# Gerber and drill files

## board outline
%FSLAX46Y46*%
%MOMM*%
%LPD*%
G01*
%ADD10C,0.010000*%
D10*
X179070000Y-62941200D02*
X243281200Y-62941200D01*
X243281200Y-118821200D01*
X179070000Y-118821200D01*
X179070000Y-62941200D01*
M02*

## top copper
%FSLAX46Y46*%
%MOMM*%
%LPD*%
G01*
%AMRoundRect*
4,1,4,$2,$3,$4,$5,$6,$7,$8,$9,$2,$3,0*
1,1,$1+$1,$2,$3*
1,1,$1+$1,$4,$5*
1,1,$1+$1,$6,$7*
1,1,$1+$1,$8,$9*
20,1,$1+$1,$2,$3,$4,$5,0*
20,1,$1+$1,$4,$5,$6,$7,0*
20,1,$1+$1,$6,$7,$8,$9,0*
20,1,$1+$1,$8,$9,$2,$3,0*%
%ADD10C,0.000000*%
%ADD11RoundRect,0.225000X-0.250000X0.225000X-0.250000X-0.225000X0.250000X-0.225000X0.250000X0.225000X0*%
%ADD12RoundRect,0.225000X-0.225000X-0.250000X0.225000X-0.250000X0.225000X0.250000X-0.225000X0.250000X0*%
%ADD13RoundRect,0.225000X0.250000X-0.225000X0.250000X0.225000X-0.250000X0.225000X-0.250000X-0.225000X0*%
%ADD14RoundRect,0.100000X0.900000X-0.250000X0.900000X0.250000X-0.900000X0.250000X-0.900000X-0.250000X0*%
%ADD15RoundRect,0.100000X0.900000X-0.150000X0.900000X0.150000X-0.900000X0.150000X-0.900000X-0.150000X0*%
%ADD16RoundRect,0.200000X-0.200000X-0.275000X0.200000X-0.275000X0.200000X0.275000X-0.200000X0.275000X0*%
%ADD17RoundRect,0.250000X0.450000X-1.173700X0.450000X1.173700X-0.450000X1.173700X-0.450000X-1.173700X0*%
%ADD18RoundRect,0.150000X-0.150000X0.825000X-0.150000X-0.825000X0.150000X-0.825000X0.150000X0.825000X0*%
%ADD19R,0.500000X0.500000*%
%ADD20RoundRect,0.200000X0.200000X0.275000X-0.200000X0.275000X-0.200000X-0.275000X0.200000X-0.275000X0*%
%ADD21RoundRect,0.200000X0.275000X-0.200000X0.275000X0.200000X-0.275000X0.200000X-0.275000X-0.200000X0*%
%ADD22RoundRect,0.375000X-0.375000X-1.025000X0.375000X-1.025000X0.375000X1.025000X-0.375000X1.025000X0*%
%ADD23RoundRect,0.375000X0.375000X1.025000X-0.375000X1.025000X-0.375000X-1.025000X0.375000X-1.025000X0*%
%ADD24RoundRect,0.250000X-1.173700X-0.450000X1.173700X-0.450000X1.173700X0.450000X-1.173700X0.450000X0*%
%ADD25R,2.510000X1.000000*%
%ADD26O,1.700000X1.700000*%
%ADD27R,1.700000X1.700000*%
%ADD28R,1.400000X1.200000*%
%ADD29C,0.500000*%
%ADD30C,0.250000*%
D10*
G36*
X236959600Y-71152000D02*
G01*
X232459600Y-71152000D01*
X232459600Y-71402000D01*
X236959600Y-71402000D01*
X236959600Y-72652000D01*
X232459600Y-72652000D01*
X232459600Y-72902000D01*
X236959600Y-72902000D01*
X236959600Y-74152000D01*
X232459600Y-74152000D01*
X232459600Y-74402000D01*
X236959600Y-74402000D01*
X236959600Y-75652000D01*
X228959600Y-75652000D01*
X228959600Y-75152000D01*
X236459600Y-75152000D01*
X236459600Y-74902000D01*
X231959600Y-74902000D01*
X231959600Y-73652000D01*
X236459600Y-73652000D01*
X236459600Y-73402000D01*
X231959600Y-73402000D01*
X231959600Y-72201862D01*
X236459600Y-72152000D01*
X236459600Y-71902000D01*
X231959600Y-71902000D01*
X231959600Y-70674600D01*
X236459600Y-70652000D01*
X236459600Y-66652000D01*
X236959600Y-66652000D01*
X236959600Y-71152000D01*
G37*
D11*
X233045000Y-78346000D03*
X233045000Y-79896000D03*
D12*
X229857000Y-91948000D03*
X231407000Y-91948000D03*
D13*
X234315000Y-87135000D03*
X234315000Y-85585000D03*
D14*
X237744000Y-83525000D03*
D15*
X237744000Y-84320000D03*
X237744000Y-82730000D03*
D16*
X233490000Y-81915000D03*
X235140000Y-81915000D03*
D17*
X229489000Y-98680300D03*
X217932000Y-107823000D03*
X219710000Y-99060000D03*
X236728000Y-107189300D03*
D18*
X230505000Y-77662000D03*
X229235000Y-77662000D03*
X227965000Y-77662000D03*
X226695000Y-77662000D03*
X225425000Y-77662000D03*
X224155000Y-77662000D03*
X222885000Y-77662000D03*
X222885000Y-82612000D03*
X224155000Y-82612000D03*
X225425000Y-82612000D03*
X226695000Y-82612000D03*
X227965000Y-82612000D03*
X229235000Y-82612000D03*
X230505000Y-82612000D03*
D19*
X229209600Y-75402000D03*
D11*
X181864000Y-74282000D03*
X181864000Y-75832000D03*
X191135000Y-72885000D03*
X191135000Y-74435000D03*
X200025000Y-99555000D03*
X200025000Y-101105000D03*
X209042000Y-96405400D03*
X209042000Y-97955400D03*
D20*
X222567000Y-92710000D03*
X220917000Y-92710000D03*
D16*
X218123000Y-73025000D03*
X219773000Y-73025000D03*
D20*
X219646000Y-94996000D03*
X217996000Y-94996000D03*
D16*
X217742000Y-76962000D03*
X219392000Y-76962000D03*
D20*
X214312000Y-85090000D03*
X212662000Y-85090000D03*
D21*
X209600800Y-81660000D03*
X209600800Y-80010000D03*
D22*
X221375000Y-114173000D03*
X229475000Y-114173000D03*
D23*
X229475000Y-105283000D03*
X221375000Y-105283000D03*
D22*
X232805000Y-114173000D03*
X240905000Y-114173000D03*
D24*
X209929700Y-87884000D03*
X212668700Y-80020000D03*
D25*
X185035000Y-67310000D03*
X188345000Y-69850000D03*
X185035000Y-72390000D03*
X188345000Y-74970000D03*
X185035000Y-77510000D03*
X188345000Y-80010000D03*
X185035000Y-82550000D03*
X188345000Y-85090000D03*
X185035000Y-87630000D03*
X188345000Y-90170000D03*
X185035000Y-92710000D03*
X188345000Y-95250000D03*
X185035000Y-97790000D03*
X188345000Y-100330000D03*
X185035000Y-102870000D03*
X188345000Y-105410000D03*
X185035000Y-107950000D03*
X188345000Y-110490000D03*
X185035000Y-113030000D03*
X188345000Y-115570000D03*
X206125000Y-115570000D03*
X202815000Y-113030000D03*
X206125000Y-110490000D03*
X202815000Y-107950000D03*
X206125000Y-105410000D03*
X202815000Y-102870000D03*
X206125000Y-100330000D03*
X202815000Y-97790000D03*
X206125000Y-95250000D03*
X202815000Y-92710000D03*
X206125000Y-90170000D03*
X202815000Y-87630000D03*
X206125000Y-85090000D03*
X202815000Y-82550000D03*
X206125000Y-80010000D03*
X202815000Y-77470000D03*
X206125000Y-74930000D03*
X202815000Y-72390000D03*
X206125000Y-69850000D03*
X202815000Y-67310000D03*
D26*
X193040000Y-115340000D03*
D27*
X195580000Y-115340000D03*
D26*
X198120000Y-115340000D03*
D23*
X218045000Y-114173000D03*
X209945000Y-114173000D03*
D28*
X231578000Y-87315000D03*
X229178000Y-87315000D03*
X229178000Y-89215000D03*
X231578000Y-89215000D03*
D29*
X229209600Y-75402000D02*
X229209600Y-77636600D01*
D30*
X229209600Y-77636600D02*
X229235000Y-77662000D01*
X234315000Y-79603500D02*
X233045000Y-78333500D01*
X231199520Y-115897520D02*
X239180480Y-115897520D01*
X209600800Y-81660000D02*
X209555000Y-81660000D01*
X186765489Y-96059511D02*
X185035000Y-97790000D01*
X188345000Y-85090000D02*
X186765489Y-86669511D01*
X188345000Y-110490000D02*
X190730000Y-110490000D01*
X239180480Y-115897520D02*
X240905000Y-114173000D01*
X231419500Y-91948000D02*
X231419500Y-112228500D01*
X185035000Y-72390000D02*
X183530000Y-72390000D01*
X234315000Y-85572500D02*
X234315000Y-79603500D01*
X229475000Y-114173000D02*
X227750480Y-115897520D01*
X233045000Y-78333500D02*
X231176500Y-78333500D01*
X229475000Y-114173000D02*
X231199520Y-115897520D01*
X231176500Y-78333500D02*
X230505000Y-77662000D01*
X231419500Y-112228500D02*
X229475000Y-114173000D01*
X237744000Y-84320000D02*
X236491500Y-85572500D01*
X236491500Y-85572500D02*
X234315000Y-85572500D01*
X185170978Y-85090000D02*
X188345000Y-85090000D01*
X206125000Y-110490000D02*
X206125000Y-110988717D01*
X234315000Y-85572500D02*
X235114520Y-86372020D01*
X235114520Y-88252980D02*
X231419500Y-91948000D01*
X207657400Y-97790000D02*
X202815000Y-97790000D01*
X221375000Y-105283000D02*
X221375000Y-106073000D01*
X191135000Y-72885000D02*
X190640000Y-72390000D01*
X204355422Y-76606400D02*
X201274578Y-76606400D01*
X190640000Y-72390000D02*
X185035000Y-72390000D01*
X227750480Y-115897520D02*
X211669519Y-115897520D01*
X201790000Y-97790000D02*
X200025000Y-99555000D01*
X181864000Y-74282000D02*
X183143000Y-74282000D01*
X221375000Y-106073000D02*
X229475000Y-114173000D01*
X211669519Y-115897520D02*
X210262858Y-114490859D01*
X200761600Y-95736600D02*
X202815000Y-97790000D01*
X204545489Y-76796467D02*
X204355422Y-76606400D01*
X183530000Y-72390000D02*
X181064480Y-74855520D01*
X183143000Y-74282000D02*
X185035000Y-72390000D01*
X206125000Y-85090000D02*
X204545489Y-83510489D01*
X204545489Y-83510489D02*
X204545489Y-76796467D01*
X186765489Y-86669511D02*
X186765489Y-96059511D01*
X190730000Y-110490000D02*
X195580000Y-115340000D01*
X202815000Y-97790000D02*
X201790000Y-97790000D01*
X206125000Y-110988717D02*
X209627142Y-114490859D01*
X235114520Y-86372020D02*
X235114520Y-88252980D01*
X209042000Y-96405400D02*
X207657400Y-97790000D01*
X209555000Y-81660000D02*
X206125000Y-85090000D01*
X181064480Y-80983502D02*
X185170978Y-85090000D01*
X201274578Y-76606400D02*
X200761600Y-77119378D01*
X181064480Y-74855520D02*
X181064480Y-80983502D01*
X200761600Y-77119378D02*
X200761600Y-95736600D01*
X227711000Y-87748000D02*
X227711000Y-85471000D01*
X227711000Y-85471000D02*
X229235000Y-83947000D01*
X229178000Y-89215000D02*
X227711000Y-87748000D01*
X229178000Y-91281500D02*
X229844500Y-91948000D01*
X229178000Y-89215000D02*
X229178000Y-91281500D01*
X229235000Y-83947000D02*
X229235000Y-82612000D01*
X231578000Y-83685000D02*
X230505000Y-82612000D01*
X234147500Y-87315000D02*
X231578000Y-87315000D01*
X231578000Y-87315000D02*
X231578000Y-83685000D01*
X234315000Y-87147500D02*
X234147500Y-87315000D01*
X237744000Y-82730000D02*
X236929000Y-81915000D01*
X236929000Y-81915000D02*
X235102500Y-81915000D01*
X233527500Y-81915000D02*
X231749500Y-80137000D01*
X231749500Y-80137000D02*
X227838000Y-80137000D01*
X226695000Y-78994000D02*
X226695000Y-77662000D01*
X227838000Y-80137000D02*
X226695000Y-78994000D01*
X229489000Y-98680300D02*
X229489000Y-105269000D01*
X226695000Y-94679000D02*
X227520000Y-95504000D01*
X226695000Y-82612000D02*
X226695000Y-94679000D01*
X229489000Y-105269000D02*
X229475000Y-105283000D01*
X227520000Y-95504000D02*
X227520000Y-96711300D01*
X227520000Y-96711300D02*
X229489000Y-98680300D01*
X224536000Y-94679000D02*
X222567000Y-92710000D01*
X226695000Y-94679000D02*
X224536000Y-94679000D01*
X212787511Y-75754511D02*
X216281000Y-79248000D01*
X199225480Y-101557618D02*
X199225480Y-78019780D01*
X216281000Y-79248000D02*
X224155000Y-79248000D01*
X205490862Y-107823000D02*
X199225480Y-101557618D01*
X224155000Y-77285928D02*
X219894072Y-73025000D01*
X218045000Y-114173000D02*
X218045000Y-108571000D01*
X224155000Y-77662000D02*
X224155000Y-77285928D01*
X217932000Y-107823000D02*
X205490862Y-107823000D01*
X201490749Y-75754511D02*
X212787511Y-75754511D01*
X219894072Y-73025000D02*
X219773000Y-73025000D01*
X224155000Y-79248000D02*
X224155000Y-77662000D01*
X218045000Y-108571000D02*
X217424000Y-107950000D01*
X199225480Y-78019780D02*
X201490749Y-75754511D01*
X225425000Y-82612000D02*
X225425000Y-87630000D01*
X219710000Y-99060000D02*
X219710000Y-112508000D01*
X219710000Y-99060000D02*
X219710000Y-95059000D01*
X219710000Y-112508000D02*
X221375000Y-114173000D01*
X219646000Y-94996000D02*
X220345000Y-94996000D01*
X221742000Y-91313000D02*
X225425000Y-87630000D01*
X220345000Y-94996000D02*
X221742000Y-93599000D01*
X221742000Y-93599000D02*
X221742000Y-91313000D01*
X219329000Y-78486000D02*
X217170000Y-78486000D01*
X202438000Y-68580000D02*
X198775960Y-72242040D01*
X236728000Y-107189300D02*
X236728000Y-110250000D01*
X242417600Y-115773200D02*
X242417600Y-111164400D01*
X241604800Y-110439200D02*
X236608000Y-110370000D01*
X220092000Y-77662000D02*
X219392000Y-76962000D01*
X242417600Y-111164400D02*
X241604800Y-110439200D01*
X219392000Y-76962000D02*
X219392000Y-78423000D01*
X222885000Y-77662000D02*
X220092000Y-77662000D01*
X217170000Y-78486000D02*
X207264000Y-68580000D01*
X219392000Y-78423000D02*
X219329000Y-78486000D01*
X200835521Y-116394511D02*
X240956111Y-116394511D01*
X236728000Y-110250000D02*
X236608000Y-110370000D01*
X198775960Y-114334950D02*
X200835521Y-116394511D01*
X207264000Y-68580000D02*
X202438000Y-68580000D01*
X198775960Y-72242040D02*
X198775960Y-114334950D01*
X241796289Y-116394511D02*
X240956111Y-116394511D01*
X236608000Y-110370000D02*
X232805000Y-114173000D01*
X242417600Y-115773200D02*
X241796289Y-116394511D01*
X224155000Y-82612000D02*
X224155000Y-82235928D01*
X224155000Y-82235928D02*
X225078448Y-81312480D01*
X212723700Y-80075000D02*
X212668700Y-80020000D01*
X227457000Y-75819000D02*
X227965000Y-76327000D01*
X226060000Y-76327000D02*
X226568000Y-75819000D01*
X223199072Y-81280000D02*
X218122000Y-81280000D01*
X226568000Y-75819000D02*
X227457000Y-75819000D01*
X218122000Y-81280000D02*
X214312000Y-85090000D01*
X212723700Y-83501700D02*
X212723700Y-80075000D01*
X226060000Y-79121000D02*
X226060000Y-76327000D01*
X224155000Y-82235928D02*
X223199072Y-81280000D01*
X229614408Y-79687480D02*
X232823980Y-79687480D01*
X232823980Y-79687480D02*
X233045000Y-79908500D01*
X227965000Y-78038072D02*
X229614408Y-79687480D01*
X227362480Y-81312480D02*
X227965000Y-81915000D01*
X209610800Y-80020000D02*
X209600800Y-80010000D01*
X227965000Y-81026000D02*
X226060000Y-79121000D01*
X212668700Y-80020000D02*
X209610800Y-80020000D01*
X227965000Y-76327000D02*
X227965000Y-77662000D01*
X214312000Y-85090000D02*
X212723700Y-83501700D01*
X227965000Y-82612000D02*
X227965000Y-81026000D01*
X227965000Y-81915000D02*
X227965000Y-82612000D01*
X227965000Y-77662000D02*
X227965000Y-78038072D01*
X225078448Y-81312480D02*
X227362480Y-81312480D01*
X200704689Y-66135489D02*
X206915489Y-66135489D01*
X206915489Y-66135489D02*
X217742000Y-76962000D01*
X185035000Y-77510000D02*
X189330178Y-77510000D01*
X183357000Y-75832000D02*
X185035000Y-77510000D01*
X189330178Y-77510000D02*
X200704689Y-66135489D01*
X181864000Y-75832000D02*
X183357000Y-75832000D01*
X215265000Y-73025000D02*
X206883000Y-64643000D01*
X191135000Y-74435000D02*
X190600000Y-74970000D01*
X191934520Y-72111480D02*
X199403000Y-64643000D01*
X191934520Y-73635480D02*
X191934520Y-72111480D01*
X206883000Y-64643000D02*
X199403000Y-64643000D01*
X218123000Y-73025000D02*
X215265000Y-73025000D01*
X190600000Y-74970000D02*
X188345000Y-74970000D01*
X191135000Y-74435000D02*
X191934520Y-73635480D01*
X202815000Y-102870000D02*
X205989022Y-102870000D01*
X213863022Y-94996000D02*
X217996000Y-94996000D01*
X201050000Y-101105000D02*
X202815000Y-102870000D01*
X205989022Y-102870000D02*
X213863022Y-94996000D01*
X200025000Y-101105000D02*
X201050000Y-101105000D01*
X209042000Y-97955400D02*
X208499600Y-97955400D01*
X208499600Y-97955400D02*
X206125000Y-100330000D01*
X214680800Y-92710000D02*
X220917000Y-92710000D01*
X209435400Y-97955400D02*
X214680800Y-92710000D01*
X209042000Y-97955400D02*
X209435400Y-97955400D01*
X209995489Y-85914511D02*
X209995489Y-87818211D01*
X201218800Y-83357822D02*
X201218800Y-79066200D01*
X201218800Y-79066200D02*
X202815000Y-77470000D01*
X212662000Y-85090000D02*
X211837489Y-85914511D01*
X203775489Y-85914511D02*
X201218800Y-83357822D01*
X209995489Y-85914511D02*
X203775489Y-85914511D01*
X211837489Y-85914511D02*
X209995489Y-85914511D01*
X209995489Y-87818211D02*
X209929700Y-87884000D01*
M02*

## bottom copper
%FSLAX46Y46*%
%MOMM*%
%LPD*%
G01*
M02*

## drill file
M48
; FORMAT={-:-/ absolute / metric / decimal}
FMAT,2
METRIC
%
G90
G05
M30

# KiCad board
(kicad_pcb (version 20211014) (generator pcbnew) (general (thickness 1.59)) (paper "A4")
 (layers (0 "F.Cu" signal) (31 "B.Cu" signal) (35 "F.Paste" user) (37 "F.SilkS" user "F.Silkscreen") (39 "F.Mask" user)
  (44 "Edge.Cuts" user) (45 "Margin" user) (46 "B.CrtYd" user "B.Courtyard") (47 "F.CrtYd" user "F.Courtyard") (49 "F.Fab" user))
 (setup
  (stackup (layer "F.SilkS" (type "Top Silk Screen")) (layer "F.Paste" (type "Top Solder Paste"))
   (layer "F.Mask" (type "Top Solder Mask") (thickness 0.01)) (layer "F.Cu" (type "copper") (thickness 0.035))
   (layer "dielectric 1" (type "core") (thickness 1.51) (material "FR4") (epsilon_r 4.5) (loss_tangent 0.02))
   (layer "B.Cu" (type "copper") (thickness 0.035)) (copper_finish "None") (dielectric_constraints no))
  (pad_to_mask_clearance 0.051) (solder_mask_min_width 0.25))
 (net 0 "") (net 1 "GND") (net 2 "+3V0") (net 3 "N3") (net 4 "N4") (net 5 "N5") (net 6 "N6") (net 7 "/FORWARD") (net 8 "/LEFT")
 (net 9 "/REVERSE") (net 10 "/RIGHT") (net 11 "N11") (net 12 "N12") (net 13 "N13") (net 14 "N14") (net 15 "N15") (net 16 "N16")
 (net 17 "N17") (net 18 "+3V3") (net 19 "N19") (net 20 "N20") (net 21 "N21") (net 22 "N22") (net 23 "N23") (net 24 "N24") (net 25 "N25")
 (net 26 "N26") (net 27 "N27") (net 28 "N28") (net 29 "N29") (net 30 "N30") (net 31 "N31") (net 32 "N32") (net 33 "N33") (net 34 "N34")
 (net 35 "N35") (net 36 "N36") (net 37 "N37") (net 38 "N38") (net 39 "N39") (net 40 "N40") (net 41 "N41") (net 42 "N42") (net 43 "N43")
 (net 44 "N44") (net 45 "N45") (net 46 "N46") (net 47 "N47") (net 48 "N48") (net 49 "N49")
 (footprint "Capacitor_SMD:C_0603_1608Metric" (layer "F.Cu") (at 233.045 79.121 -90)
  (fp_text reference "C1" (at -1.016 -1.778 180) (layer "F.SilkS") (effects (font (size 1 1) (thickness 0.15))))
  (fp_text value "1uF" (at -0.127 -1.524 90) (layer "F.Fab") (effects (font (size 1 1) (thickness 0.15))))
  (pad "1" smd roundrect locked (at -0.775 0 270) (size 0.9 0.95) (layers "F.Cu" "F.Paste" "F.Mask") (roundrect_rratio 0.25) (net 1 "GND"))
  (pad "2" smd roundrect locked (at 0.775 0 270) (size 0.9 0.95) (layers "F.Cu" "F.Paste" "F.Mask") (roundrect_rratio 0.25) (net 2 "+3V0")))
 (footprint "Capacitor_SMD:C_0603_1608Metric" (layer "F.Cu") (at 230.632 91.948)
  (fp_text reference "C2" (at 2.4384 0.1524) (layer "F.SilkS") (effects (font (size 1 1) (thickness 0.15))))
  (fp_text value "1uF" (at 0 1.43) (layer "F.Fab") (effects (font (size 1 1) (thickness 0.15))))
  (pad "1" smd roundrect locked (at -0.775 0) (size 0.9 0.95) (layers "F.Cu" "F.Paste" "F.Mask") (roundrect_rratio 0.25) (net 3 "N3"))
  (pad "2" smd roundrect locked (at 0.775 0) (size 0.9 0.95) (layers "F.Cu" "F.Paste" "F.Mask") (roundrect_rratio 0.25) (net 1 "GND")))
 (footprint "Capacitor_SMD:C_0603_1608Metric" (layer "F.Cu") (at 234.315 86.36 90)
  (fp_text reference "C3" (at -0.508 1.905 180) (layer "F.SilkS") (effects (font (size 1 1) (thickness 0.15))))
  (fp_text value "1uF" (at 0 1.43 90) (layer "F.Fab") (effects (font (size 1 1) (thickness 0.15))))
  (pad "1" smd roundrect locked (at -0.775 0 90) (size 0.9 0.95) (layers "F.Cu" "F.Paste" "F.Mask") (roundrect_rratio 0.25) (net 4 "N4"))
  (pad "2" smd roundrect locked (at 0.775 0 90) (size 0.9 0.95) (layers "F.Cu" "F.Paste" "F.Mask") (roundrect_rratio 0.25) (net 1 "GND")))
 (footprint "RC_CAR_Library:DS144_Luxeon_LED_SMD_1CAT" (layer "F.Cu") (at 237.744 83.525 90)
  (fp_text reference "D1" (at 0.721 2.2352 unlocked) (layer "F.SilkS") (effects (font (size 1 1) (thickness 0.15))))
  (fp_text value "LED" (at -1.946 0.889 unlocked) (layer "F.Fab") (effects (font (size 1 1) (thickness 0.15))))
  (pad "" smd roundrect (at 0 0 90) (size 0.7 2) (layers "F.Cu" "F.Paste" "F.Mask") (roundrect_rratio 0.1428571429) (zone_connect 1))
  (pad "1" smd roundrect (at -0.795 0 90) (size 0.5 2) (layers "F.Cu" "F.Paste" "F.Mask") (roundrect_rratio 0.2) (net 1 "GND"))
  (pad "2" smd roundrect (at 0.795 0 90) (size 0.5 2) (layers "F.Cu" "F.Paste" "F.Mask") (roundrect_rratio 0.2) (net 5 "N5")))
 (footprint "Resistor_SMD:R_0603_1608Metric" (layer "F.Cu") (at 234.315 81.915)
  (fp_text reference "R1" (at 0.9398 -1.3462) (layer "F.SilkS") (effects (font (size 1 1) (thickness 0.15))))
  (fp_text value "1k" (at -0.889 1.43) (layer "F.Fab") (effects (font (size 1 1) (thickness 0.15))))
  (pad "1" smd roundrect locked (at -0.825 0) (size 0.8 0.95) (layers "F.Cu" "F.Paste" "F.Mask") (roundrect_rratio 0.25) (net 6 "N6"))
  (pad "2" smd roundrect locked (at 0.825 0) (size 0.8 0.95) (layers "F.Cu" "F.Paste" "F.Mask") (roundrect_rratio 0.25) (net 5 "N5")))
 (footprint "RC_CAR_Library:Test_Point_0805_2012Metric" (layer "F.Cu") (at 229.489 98.679 90)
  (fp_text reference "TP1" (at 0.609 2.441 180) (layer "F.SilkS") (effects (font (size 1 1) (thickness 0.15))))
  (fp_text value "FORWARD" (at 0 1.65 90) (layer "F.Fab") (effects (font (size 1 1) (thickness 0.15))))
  (pad "1" smd roundrect (at -0.0013 0 90) (size 2.8474 1.4) (layers "F.Cu" "F.Paste" "F.Mask") (roundrect_rratio 0.1785714286)
   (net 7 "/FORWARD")))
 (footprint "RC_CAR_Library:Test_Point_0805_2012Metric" (layer "F.Cu") (at 217.932 107.8217 90)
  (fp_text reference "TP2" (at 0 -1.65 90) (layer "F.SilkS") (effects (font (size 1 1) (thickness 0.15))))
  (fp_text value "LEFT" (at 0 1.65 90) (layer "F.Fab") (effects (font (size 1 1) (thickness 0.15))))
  (pad "1" smd roundrect (at -0.0013 0 90) (size 2.8474 1.4) (layers "F.Cu" "F.Paste" "F.Mask") (roundrect_rratio 0.1785714286)
   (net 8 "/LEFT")))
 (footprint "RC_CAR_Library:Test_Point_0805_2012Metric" (layer "F.Cu") (at 219.71 99.0587 90)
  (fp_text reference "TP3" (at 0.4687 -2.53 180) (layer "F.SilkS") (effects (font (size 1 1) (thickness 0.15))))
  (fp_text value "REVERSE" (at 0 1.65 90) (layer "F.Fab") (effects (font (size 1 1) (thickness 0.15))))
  (pad "1" smd roundrect (at -0.0013 0 90) (size 2.8474 1.4) (layers "F.Cu" "F.Paste" "F.Mask") (roundrect_rratio 0.1785714286)
   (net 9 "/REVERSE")))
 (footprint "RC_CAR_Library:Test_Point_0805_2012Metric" (layer "F.Cu") (at 236.728 107.188 90)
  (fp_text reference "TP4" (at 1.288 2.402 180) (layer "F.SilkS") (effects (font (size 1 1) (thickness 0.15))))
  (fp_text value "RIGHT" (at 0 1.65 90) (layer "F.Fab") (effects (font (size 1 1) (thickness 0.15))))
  (pad "1" smd roundrect (at -0.0013 0 90) (size 2.8474 1.4) (layers "F.Cu" "F.Paste" "F.Mask") (roundrect_rratio 0.1785714286)
   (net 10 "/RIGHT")))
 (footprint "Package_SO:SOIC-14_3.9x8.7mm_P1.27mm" (layer "F.Cu") (at 226.695 80.137 -90)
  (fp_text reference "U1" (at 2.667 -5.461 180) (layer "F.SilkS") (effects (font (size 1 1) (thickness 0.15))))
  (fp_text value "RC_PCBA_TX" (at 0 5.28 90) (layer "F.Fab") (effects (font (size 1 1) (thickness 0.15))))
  (pad "1" smd roundrect locked (at -2.475 -3.81 270) (size 1.95 0.6) (layers "F.Cu" "F.Paste" "F.Mask") (roundrect_rratio 0.25)
   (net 1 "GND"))
  (pad "2" smd roundrect locked (at -2.475 -2.54 270) (size 1.95 0.6) (layers "F.Cu" "F.Paste" "F.Mask") (roundrect_rratio 0.25)
   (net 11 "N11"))
  (pad "3" smd roundrect locked (at -2.475 -1.27 270) (size 1.95 0.6) (layers "F.Cu" "F.Paste" "F.Mask") (roundrect_rratio 0.25)
   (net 2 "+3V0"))
  (pad "4" smd roundrect locked (at -2.475 0 270) (size 1.95 0.6) (layers "F.Cu" "F.Paste" "F.Mask") (roundrect_rratio 0.25) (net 6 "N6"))
  (pad "5" smd roundrect locked (at -2.475 1.27 270) (size 1.95 0.6) (layers "F.Cu" "F.Paste" "F.Mask") (roundrect_rratio 0.25)
   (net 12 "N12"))
  (pad "6" smd roundrect locked (at -2.475 2.54 270) (size 1.95 0.6) (layers "F.Cu" "F.Paste" "F.Mask") (roundrect_rratio 0.25)
   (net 8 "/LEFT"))
  (pad "7" smd roundrect locked (at -2.475 3.81 270) (size 1.95 0.6) (layers "F.Cu" "F.Paste" "F.Mask") (roundrect_rratio 0.25)
   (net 10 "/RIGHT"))
  (pad "8" smd roundrect locked (at 2.475 3.81 270) (size 1.95 0.6) (layers "F.Cu" "F.Paste" "F.Mask") (roundrect_rratio 0.25)
   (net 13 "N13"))
  (pad "9" smd roundrect locked (at 2.475 2.54 270) (size 1.95 0.6) (layers "F.Cu" "F.Paste" "F.Mask") (roundrect_rratio 0.25)
   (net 2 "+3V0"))
  (pad "10" smd roundrect locked (at 2.475 1.27 270) (size 1.95 0.6) (layers "F.Cu" "F.Paste" "F.Mask") (roundrect_rratio 0.25)
   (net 9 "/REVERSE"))
  (pad "11" smd roundrect locked (at 2.475 0 270) (size 1.95 0.6) (layers "F.Cu" "F.Paste" "F.Mask") (roundrect_rratio 0.25)
   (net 7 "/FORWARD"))
  (pad "12" smd roundrect locked (at 2.475 -1.27 270) (size 1.95 0.6) (layers "F.Cu" "F.Paste" "F.Mask") (roundrect_rratio 0.25)
   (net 2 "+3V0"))
  (pad "13" smd roundrect locked (at 2.475 -2.54 270) (size 1.95 0.6) (layers "F.Cu" "F.Paste" "F.Mask") (roundrect_rratio 0.25)
   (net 3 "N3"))
  (pad "14" smd roundrect locked (at 2.475 -3.81 270) (size 1.95 0.6) (layers "F.Cu" "F.Paste" "F.Mask") (roundrect_rratio 0.25)
   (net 4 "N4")))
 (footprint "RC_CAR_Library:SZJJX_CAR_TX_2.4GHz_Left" (layer "F.Cu") (at 229.2096 73.152 -90)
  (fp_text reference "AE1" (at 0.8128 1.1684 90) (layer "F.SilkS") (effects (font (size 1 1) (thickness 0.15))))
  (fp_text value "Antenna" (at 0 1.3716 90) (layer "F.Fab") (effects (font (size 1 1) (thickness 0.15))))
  (fp_poly
   (pts (xy -2 -7.75) (xy -2 -3.25) (xy -1.75 -3.25) (xy -1.75 -7.75) (xy -0.5 -7.75) (xy -0.5 -3.25) (xy -0.25 -3.25) (xy -0.25 -7.75)
    (xy 1 -7.75) (xy 1 -3.25) (xy 1.25 -3.25) (xy 1.25 -7.75) (xy 2.5 -7.75) (xy 2.5 0.25) (xy 2 0.25) (xy 2 -7.25) (xy 1.75 -7.25)
    (xy 1.75 -2.75) (xy 0.5 -2.75) (xy 0.5 -7.25) (xy 0.25 -7.25) (xy 0.25 -2.75) (xy -0.950138 -2.75) (xy -1 -7.25) (xy -1.25 -7.25)
    (xy -1.25 -2.75) (xy -2.4774 -2.75) (xy -2.5 -7.25) (xy -6.5 -7.25) (xy -6.5 -7.75))
   (layer "F.Cu") (width 0) (fill solid))
  (pad "1" connect rect (at 2.25 0 270) (size 0.5 0.5) (layers "F.Cu") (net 11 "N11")))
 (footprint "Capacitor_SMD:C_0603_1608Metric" (layer "F.Cu") (at 181.864 75.057 -90)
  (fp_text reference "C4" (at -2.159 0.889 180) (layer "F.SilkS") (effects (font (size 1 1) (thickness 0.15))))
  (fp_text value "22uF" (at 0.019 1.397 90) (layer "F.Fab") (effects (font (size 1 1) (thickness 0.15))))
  (pad "1" smd roundrect locked (at -0.775 0 270) (size 0.9 0.95) (layers "F.Cu" "F.Paste" "F.Mask") (roundrect_rratio 0.25) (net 1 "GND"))
  (pad "2" smd roundrect locked (at 0.775 0 270) (size 0.9 0.95) (layers "F.Cu" "F.Paste" "F.Mask") (roundrect_rratio 0.25) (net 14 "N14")))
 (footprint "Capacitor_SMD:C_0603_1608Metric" (layer "F.Cu") (at 191.135 73.66 -90)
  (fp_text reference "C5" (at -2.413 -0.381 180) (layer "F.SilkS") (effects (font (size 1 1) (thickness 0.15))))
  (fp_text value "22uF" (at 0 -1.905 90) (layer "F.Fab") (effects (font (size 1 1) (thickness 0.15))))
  (pad "1" smd roundrect locked (at -0.775 0 270) (size 0.9 0.95) (layers "F.Cu" "F.Paste" "F.Mask") (roundrect_rratio 0.25) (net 1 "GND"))
  (pad "2" smd roundrect locked (at 0.775 0 270) (size 0.9 0.95) (layers "F.Cu" "F.Paste" "F.Mask") (roundrect_rratio 0.25) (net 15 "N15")))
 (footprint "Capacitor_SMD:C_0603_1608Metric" (layer "F.Cu") (at 200.025 100.33 -90)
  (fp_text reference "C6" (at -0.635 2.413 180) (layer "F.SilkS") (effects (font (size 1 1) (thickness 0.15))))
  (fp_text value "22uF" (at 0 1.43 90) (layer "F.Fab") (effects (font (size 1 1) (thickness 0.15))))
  (pad "1" smd roundrect locked (at -0.775 0 270) (size 0.9 0.95) (layers "F.Cu" "F.Paste" "F.Mask") (roundrect_rratio 0.25) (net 1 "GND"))
  (pad "2" smd roundrect locked (at 0.775 0 270) (size 0.9 0.95) (layers "F.Cu" "F.Paste" "F.Mask") (roundrect_rratio 0.25) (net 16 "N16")))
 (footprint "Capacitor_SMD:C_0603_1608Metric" (layer "F.Cu") (at 209.042 97.1804 -90)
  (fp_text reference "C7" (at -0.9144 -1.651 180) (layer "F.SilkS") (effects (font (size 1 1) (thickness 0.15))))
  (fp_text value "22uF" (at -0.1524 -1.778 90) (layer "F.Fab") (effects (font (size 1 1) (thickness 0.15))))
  (pad "1" smd roundrect locked (at -0.775 0 270) (size 0.9 0.95) (layers "F.Cu" "F.Paste" "F.Mask") (roundrect_rratio 0.25) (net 1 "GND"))
  (pad "2" smd roundrect locked (at 0.775 0 270) (size 0.9 0.95) (layers "F.Cu" "F.Paste" "F.Mask") (roundrect_rratio 0.25) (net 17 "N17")))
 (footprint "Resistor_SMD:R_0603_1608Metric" (layer "F.Cu") (at 221.742 92.71 180)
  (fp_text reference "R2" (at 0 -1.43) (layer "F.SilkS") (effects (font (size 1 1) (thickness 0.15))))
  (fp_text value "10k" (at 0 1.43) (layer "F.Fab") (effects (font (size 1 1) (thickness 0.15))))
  (pad "1" smd roundrect locked (at -0.825 0 180) (size 0.8 0.95) (layers "F.Cu" "F.Paste" "F.Mask") (roundrect_rratio 0.25)
   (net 7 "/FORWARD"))
  (pad "2" smd roundrect locked (at 0.825 0 180) (size 0.8 0.95) (layers "F.Cu" "F.Paste" "F.Mask") (roundrect_rratio 0.25) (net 17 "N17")))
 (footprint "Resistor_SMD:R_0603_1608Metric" (layer "F.Cu") (at 218.948 73.025)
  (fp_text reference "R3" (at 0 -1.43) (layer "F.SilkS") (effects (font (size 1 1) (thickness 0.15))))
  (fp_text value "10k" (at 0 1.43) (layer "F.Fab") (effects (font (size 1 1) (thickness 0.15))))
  (pad "1" smd roundrect locked (at -0.825 0) (size 0.8 0.95) (layers "F.Cu" "F.Paste" "F.Mask") (roundrect_rratio 0.25) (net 15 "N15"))
  (pad "2" smd roundrect locked (at 0.825 0) (size 0.8 0.95) (layers "F.Cu" "F.Paste" "F.Mask") (roundrect_rratio 0.25) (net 8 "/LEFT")))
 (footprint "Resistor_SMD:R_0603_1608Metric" (layer "F.Cu") (at 218.821 94.996 180)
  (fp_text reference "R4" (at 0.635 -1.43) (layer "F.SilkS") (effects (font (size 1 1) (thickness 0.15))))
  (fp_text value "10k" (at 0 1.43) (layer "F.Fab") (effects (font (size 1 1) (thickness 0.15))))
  (pad "1" smd roundrect locked (at -0.825 0 180) (size 0.8 0.95) (layers "F.Cu" "F.Paste" "F.Mask") (roundrect_rratio 0.25)
   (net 9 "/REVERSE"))
  (pad "2" smd roundrect locked (at 0.825 0 180) (size 0.8 0.95) (layers "F.Cu" "F.Paste" "F.Mask") (roundrect_rratio 0.25) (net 16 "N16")))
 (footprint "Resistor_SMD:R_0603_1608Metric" (layer "F.Cu") (at 218.567 76.962)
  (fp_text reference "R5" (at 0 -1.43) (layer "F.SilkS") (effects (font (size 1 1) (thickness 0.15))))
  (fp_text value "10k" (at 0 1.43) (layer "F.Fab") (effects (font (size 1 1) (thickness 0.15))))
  (pad "1" smd roundrect locked (at -0.825 0) (size 0.8 0.95) (layers "F.Cu" "F.Paste" "F.Mask") (roundrect_rratio 0.25) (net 14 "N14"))
  (pad "2" smd roundrect locked (at 0.825 0) (size 0.8 0.95) (layers "F.Cu" "F.Paste" "F.Mask") (roundrect_rratio 0.25) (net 10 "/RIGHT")))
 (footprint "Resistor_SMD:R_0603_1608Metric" (layer "F.Cu") (at 213.487 85.09 180)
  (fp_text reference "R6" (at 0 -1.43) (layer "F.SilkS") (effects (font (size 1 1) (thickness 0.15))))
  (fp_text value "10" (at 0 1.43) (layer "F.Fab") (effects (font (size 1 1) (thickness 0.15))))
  (pad "1" smd roundrect locked (at -0.825 0 180) (size 0.8 0.95) (layers "F.Cu" "F.Paste" "F.Mask") (roundrect_rratio 0.25) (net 2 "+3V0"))
  (pad "2" smd roundrect locked (at 0.825 0 180) (size 0.8 0.95) (layers "F.Cu" "F.Paste" "F.Mask") (roundrect_rratio 0.25) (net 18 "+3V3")))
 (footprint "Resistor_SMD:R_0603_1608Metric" (layer "F.Cu") (at 209.6008 80.835 90)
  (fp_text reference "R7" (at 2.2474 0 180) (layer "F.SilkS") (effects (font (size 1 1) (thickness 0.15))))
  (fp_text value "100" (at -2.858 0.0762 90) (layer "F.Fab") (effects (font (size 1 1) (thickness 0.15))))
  (pad "1" smd roundrect locked (at -0.825 0 90) (size 0.8 0.95) (layers "F.Cu" "F.Paste" "F.Mask") (roundrect_rratio 0.25) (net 1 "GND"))
  (pad "2" smd roundrect locked (at 0.825 0 90) (size 0.8 0.95) (layers "F.Cu" "F.Paste" "F.Mask") (roundrect_rratio 0.25) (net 2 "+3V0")))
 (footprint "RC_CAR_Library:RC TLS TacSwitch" (layer "F.Cu") (at 225.425 114.173)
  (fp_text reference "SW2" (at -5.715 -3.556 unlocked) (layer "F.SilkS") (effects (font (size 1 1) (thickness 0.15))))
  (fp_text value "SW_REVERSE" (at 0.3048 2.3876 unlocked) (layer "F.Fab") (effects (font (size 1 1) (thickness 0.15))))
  (pad "1" smd roundrect (at -4.05 0) (size 1.5 2.8) (layers "F.Cu" "F.Paste" "F.Mask") (roundrect_rratio 0.25) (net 9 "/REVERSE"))
  (pad "2" smd roundrect (at 4.05 0) (size 1.5 2.8) (layers "F.Cu" "F.Paste" "F.Mask") (roundrect_rratio 0.25) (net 1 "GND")))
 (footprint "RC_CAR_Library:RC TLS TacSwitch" (layer "F.Cu") (at 225.425 105.283 180)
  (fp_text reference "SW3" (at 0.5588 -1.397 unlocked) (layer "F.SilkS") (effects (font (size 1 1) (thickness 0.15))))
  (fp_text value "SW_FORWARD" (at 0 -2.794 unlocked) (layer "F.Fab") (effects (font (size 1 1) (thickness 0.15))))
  (pad "1" smd roundrect (at -4.05 0 180) (size 1.5 2.8) (layers "F.Cu" "F.Paste" "F.Mask") (roundrect_rratio 0.25) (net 7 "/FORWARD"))
  (pad "2" smd roundrect (at 4.05 0 180) (size 1.5 2.8) (layers "F.Cu" "F.Paste" "F.Mask") (roundrect_rratio 0.25) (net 1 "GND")))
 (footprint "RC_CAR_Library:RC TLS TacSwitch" (layer "F.Cu") (at 236.855 114.173)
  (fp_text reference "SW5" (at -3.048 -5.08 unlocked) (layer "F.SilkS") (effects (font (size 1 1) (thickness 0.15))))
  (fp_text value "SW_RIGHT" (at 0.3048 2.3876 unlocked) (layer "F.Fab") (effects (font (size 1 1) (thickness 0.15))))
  (pad "1" smd roundrect (at -4.05 0) (size 1.5 2.8) (layers "F.Cu" "F.Paste" "F.Mask") (roundrect_rratio 0.25) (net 10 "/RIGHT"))
  (pad "2" smd roundrect (at 4.05 0) (size 1.5 2.8) (layers "F.Cu" "F.Paste" "F.Mask") (roundrect_rratio 0.25) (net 1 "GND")))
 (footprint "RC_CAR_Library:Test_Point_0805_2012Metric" (layer "F.Cu") (at 209.931 87.884)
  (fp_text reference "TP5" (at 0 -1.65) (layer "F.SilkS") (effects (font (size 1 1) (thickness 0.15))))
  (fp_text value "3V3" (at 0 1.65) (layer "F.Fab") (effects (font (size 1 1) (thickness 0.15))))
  (pad "1" smd roundrect (at -0.0013 0) (size 2.8474 1.4) (layers "F.Cu" "F.Paste" "F.Mask") (roundrect_rratio 0.1785714286) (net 18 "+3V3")))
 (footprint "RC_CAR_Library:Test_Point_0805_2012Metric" (layer "F.Cu") (at 212.67 80.02)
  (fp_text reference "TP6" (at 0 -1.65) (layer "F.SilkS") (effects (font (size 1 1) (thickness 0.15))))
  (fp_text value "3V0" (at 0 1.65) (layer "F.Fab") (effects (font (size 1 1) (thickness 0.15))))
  (pad "1" smd roundrect (at -0.0013 0) (size 2.8474 1.4) (layers "F.Cu" "F.Paste" "F.Mask") (roundrect_rratio 0.1785714286) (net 2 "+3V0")))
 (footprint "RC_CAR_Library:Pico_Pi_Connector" (layer "F.Cu") (at 195.58 91.44)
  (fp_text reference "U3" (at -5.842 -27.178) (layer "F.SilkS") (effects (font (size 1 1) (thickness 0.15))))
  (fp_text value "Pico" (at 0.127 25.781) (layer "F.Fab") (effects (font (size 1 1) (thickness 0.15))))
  (pad "1" smd rect (at -10.545 -24.13) (size 2.51 1) (layers "F.Cu" "F.Paste" "F.Mask") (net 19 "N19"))
  (pad "2" smd rect (at -7.235 -21.59) (size 2.51 1) (layers "F.Cu" "F.Paste" "F.Mask") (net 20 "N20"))
  (pad "3" smd rect (at -10.545 -19.05) (size 2.51 1) (layers "F.Cu" "F.Paste" "F.Mask") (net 1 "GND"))
  (pad "4" smd rect (at -7.235 -16.47) (size 2.51 1) (layers "F.Cu" "F.Paste" "F.Mask") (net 15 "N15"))
  (pad "5" smd rect (at -10.545 -13.93) (size 2.51 1) (layers "F.Cu" "F.Paste" "F.Mask") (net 14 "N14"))
  (pad "6" smd rect (at -7.235 -11.43) (size 2.51 1) (layers "F.Cu" "F.Paste" "F.Mask") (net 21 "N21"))
  (pad "7" smd rect (at -10.545 -8.89) (size 2.51 1) (layers "F.Cu" "F.Paste" "F.Mask") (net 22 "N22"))
  (pad "8" smd rect (at -7.235 -6.35) (size 2.51 1) (layers "F.Cu" "F.Paste" "F.Mask") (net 1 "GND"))
  (pad "9" smd rect (at -10.545 -3.81) (size 2.51 1) (layers "F.Cu" "F.Paste" "F.Mask") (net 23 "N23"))
  (pad "10" smd rect (at -7.235 -1.27) (size 2.51 1) (layers "F.Cu" "F.Paste" "F.Mask") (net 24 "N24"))
  (pad "11" smd rect (at -10.545 1.27) (size 2.51 1) (layers "F.Cu" "F.Paste" "F.Mask") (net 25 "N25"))
  (pad "12" smd rect (at -7.235 3.81) (size 2.51 1) (layers "F.Cu" "F.Paste" "F.Mask") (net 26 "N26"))
  (pad "13" smd rect (at -10.545 6.35) (size 2.51 1) (layers "F.Cu" "F.Paste" "F.Mask") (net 1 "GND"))
  (pad "14" smd rect (at -7.235 8.89) (size 2.51 1) (layers "F.Cu" "F.Paste" "F.Mask") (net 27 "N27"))
  (pad "15" smd rect (at -10.545 11.43) (size 2.51 1) (layers "F.Cu" "F.Paste" "F.Mask") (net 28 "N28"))
  (pad "16" smd rect (at -7.235 13.97) (size 2.51 1) (layers "F.Cu" "F.Paste" "F.Mask") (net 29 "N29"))
  (pad "17" smd rect (at -10.545 16.51) (size 2.51 1) (layers "F.Cu" "F.Paste" "F.Mask") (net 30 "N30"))
  (pad "18" smd rect (at -7.235 19.05) (size 2.51 1) (layers "F.Cu" "F.Paste" "F.Mask") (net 1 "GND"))
  (pad "19" smd rect (at -10.545 21.59) (size 2.51 1) (layers "F.Cu" "F.Paste" "F.Mask") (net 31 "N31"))
  (pad "20" smd rect (at -7.235 24.13) (size 2.51 1) (layers "F.Cu" "F.Paste" "F.Mask") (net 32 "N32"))
  (pad "21" smd rect (at 10.545 24.13) (size 2.51 1) (layers "F.Cu" "F.Paste" "F.Mask") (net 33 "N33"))
  (pad "22" smd rect (at 7.235 21.59) (size 2.51 1) (layers "F.Cu" "F.Paste" "F.Mask") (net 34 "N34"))
  (pad "23" smd rect (at 10.545 19.05) (size 2.51 1) (layers "F.Cu" "F.Paste" "F.Mask") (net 1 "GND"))
  (pad "24" smd rect (at 7.235 16.51) (size 2.51 1) (layers "F.Cu" "F.Paste" "F.Mask") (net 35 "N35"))
  (pad "25" smd rect (at 10.545 13.97) (size 2.51 1) (layers "F.Cu" "F.Paste" "F.Mask") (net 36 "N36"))
  (pad "26" smd rect (at 7.235 11.43) (size 2.51 1) (layers "F.Cu" "F.Paste" "F.Mask") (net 16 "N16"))
  (pad "27" smd rect (at 10.545 8.89) (size 2.51 1) (layers "F.Cu" "F.Paste" "F.Mask") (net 17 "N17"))
  (pad "28" smd rect (at 7.235 6.35) (size 2.51 1) (layers "F.Cu" "F.Paste" "F.Mask") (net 1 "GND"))
  (pad "29" smd rect (at 10.545 3.81) (size 2.51 1) (layers "F.Cu" "F.Paste" "F.Mask") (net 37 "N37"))
  (pad "30" smd rect (at 7.235 1.27) (size 2.51 1) (layers "F.Cu" "F.Paste" "F.Mask") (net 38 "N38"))
  (pad "31" smd rect (at 10.545 -1.27) (size 2.51 1) (layers "F.Cu" "F.Paste" "F.Mask") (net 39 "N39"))
  (pad "32" smd rect (at 7.235 -3.81) (size 2.51 1) (layers "F.Cu" "F.Paste" "F.Mask") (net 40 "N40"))
  (pad "33" smd rect (at 10.545 -6.35) (size 2.51 1) (layers "F.Cu" "F.Paste" "F.Mask") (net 1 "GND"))
  (pad "34" smd rect (at 7.235 -8.89) (size 2.51 1) (layers "F.Cu" "F.Paste" "F.Mask") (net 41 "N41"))
  (pad "35" smd rect (at 10.545 -11.43) (size 2.51 1) (layers "F.Cu" "F.Paste" "F.Mask") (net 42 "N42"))
  (pad "36" smd rect (at 7.235 -13.97) (size 2.51 1) (layers "F.Cu" "F.Paste" "F.Mask") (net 18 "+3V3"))
  (pad "37" smd rect (at 10.545 -16.51) (size 2.51 1) (layers "F.Cu" "F.Paste" "F.Mask") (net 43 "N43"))
  (pad "38" smd rect (at 7.235 -19.05) (size 2.51 1) (layers "F.Cu" "F.Paste" "F.Mask") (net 1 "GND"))
  (pad "39" smd rect (at 10.545 -21.59) (size 2.51 1) (layers "F.Cu" "F.Paste" "F.Mask") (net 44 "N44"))
  (pad "40" smd rect (at 7.235 -24.13) (size 2.51 1) (layers "F.Cu" "F.Paste" "F.Mask") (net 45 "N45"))
  (pad "41" smd oval (at -2.54 23.9) (size 1.7 1.7) (layers "F.Cu" "F.Paste" "F.Mask") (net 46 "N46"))
  (pad "42" smd rect (at 0 23.9) (size 1.7 1.7) (layers "F.Cu" "F.Paste" "F.Mask") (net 1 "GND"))
  (pad "43" smd oval (at 2.54 23.9) (size 1.7 1.7) (layers "F.Cu" "F.Paste" "F.Mask") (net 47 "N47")))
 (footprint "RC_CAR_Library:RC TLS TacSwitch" (layer "F.Cu") (at 213.995 114.173 180)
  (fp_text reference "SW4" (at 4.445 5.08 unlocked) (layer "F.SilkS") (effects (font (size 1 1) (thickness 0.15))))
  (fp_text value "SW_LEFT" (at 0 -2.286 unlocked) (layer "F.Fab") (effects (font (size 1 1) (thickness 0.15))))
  (pad "1" smd roundrect (at -4.05 0 180) (size 1.5 2.8) (layers "F.Cu" "F.Paste" "F.Mask") (roundrect_rratio 0.25) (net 8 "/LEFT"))
  (pad "2" smd roundrect (at 4.05 0 180) (size 1.5 2.8) (layers "F.Cu" "F.Paste" "F.Mask") (roundrect_rratio 0.25) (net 1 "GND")))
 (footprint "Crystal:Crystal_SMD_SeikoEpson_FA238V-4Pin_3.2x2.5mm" (layer "F.Cu") (at 230.378 88.265 180)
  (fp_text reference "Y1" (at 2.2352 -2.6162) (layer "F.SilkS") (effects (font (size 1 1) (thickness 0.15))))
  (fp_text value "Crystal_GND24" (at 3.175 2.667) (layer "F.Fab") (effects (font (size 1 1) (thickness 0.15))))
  (pad "1" smd rect locked (at -1.2 0.95 180) (size 1.4 1.2) (layers "F.Cu" "F.Paste" "F.Mask") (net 4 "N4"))
  (pad "2" smd rect locked (at 1.2 0.95 180) (size 1.4 1.2) (layers "F.Cu" "F.Paste" "F.Mask") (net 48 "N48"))
  (pad "3" smd rect locked (at 1.2 -0.95 180) (size 1.4 1.2) (layers "F.Cu" "F.Paste" "F.Mask") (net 3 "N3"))
  (pad "4" smd rect locked (at -1.2 -0.95 180) (size 1.4 1.2) (layers "F.Cu" "F.Paste" "F.Mask") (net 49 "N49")))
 (gr_rect (start 179.07 62.9412) (end 243.2812 118.8212) (layer "Edge.Cuts") (width 0.01) (fill none))
 (segment (start 229.2096 75.402) (end 229.2096 77.6366) (width 0.5) (layer "F.Cu") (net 11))
 (segment (start 229.2096 77.6366) (end 229.235 77.662) (width 0.25) (layer "F.Cu") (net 11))
 (segment (start 234.315 79.6035) (end 233.045 78.3335) (width 0.25) (layer "F.Cu") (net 1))
 (segment (start 231.19952 115.89752) (end 239.18048 115.89752) (width 0.25) (layer "F.Cu") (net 1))
 (segment (start 209.6008 81.66) (end 209.555 81.66) (width 0.25) (layer "F.Cu") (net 1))
 (segment (start 186.765489 96.059511) (end 185.035 97.79) (width 0.25) (layer "F.Cu") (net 1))
 (segment (start 188.345 85.09) (end 186.765489 86.669511) (width 0.25) (layer "F.Cu") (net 1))
 (segment (start 188.345 110.49) (end 190.73 110.49) (width 0.25) (layer "F.Cu") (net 1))
 (segment (start 239.18048 115.89752) (end 240.905 114.173) (width 0.25) (layer "F.Cu") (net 1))
 (segment (start 231.4195 91.948) (end 231.4195 112.2285) (width 0.25) (layer "F.Cu") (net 1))
 (segment (start 185.035 72.39) (end 183.53 72.39) (width 0.25) (layer "F.Cu") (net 1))
 (segment (start 234.315 85.5725) (end 234.315 79.6035) (width 0.25) (layer "F.Cu") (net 1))
 (segment (start 229.475 114.173) (end 227.75048 115.89752) (width 0.25) (layer "F.Cu") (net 1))
 (segment (start 233.045 78.3335) (end 231.1765 78.3335) (width 0.25) (layer "F.Cu") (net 1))
 (segment (start 229.475 114.173) (end 231.19952 115.89752) (width 0.25) (layer "F.Cu") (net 1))
 (segment (start 231.1765 78.3335) (end 230.505 77.662) (width 0.25) (layer "F.Cu") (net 1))
 (segment (start 231.4195 112.2285) (end 229.475 114.173) (width 0.25) (layer "F.Cu") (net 1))
 (segment (start 237.744 84.32) (end 236.4915 85.5725) (width 0.25) (layer "F.Cu") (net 1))
 (segment (start 236.4915 85.5725) (end 234.315 85.5725) (width 0.25) (layer "F.Cu") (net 1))
 (segment (start 185.170978 85.09) (end 188.345 85.09) (width 0.25) (layer "F.Cu") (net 1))
 (segment (start 206.125 110.49) (end 206.125 110.988717) (width 0.25) (layer "F.Cu") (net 1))
 (segment (start 234.315 85.5725) (end 235.11452 86.37202) (width 0.25) (layer "F.Cu") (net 1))
 (segment (start 235.11452 88.25298) (end 231.4195 91.948) (width 0.25) (layer "F.Cu") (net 1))
 (segment (start 207.6574 97.79) (end 202.815 97.79) (width 0.25) (layer "F.Cu") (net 1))
 (segment (start 221.375 105.283) (end 221.375 106.073) (width 0.25) (layer "F.Cu") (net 1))
 (segment (start 191.135 72.885) (end 190.64 72.39) (width 0.25) (layer "F.Cu") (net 1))
 (segment (start 204.355422 76.6064) (end 201.274578 76.6064) (width 0.25) (layer "F.Cu") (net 1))
 (segment (start 190.64 72.39) (end 185.035 72.39) (width 0.25) (layer "F.Cu") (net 1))
 (segment (start 227.75048 115.89752) (end 211.669519 115.89752) (width 0.25) (layer "F.Cu") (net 1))
 (segment (start 201.79 97.79) (end 200.025 99.555) (width 0.25) (layer "F.Cu") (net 1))
 (segment (start 181.864 74.282) (end 183.143 74.282) (width 0.25) (layer "F.Cu") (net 1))
 (segment (start 221.375 106.073) (end 229.475 114.173) (width 0.25) (layer "F.Cu") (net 1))
 (segment (start 211.669519 115.89752) (end 210.262858 114.490859) (width 0.25) (layer "F.Cu") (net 1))
 (segment (start 200.7616 95.7366) (end 202.815 97.79) (width 0.25) (layer "F.Cu") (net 1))
 (segment (start 204.545489 76.796467) (end 204.355422 76.6064) (width 0.25) (layer "F.Cu") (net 1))
 (segment (start 183.53 72.39) (end 181.06448 74.85552) (width 0.25) (layer "F.Cu") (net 1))
 (segment (start 183.143 74.282) (end 185.035 72.39) (width 0.25) (layer "F.Cu") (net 1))
 (segment (start 206.125 85.09) (end 204.545489 83.510489) (width 0.25) (layer "F.Cu") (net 1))
 (segment (start 204.545489 83.510489) (end 204.545489 76.796467) (width 0.25) (layer "F.Cu") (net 1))
 (segment (start 186.765489 86.669511) (end 186.765489 96.059511) (width 0.25) (layer "F.Cu") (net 1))
 (segment (start 190.73 110.49) (end 195.58 115.34) (width 0.25) (layer "F.Cu") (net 1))
 (segment (start 202.815 97.79) (end 201.79 97.79) (width 0.25) (layer "F.Cu") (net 1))
 (segment (start 206.125 110.988717) (end 209.627142 114.490859) (width 0.25) (layer "F.Cu") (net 1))
 (segment (start 235.11452 86.37202) (end 235.11452 88.25298) (width 0.25) (layer "F.Cu") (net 1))
 (segment (start 209.042 96.4054) (end 207.6574 97.79) (width 0.25) (layer "F.Cu") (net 1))
 (segment (start 209.555 81.66) (end 206.125 85.09) (width 0.25) (layer "F.Cu") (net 1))
 (segment (start 181.06448 80.983502) (end 185.170978 85.09) (width 0.25) (layer "F.Cu") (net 1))
 (segment (start 201.274578 76.6064) (end 200.7616 77.119378) (width 0.25) (layer "F.Cu") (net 1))
 (segment (start 181.06448 74.85552) (end 181.06448 80.983502) (width 0.25) (layer "F.Cu") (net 1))
 (segment (start 200.7616 77.119378) (end 200.7616 95.7366) (width 0.25) (layer "F.Cu") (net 1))
 (segment (start 227.711 87.748) (end 227.711 85.471) (width 0.25) (layer "F.Cu") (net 3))
 (segment (start 227.711 85.471) (end 229.235 83.947) (width 0.25) (layer "F.Cu") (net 3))
 (segment (start 229.178 89.215) (end 227.711 87.748) (width 0.25) (layer "F.Cu") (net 3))
 (segment (start 229.178 91.2815) (end 229.8445 91.948) (width 0.25) (layer "F.Cu") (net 3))
 (segment (start 229.178 89.215) (end 229.178 91.2815) (width 0.25) (layer "F.Cu") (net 3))
 (segment (start 229.235 83.947) (end 229.235 82.612) (width 0.25) (layer "F.Cu") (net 3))
 (segment (start 231.578 83.685) (end 230.505 82.612) (width 0.25) (layer "F.Cu") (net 4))
 (segment (start 234.1475 87.315) (end 231.578 87.315) (width 0.25) (layer "F.Cu") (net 4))
 (segment (start 231.578 87.315) (end 231.578 83.685) (width 0.25) (layer "F.Cu") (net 4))
 (segment (start 234.315 87.1475) (end 234.1475 87.315) (width 0.25) (layer "F.Cu") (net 4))
 (segment (start 237.744 82.73) (end 236.929 81.915) (width 0.25) (layer "F.Cu") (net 5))
 (segment (start 236.929 81.915) (end 235.1025 81.915) (width 0.25) (layer "F.Cu") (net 5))
 (segment (start 233.5275 81.915) (end 231.7495 80.137) (width 0.25) (layer "F.Cu") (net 6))
 (segment (start 231.7495 80.137) (end 227.838 80.137) (width 0.25) (layer "F.Cu") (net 6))
 (segment (start 226.695 78.994) (end 226.695 77.662) (width 0.25) (layer "F.Cu") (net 6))
 (segment (start 227.838 80.137) (end 226.695 78.994) (width 0.25) (layer "F.Cu") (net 6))
 (segment (start 229.489 98.6803) (end 229.489 105.269) (width 0.25) (layer "F.Cu") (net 7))
 (segment (start 226.695 94.679) (end 227.52 95.504) (width 0.25) (layer "F.Cu") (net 7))
 (segment (start 226.695 82.612) (end 226.695 94.679) (width 0.25) (layer "F.Cu") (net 7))
 (segment (start 229.489 105.269) (end 229.475 105.283) (width 0.25) (layer "F.Cu") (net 7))
 (segment (start 227.52 95.504) (end 227.52 96.7113) (width 0.25) (layer "F.Cu") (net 7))
 (segment (start 227.52 96.7113) (end 229.489 98.6803) (width 0.25) (layer "F.Cu") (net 7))
 (segment (start 224.536 94.679) (end 222.567 92.71) (width 0.25) (layer "F.Cu") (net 7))
 (segment (start 226.695 94.679) (end 224.536 94.679) (width 0.25) (layer "F.Cu") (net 7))
 (segment (start 212.787511 75.754511) (end 216.281 79.248) (width 0.25) (layer "F.Cu") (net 8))
 (segment (start 199.22548 101.557618) (end 199.22548 78.01978) (width 0.25) (layer "F.Cu") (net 8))
 (segment (start 216.281 79.248) (end 224.155 79.248) (width 0.25) (layer "F.Cu") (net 8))
 (segment (start 205.490862 107.823) (end 199.22548 101.557618) (width 0.25) (layer "F.Cu") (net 8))
 (segment (start 224.155 77.285928) (end 219.894072 73.025) (width 0.25) (layer "F.Cu") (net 8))
 (segment (start 218.045 114.173) (end 218.045 108.571) (width 0.25) (layer "F.Cu") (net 8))
 (segment (start 224.155 77.662) (end 224.155 77.285928) (width 0.25) (layer "F.Cu") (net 8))
 (segment (start 217.932 107.823) (end 205.490862 107.823) (width 0.25) (layer "F.Cu") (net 8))
 (segment (start 201.490749 75.754511) (end 212.787511 75.754511) (width 0.25) (layer "F.Cu") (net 8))
 (segment (start 219.894072 73.025) (end 219.773 73.025) (width 0.25) (layer "F.Cu") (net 8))
 (segment (start 224.155 79.248) (end 224.155 77.662) (width 0.25) (layer "F.Cu") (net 8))
 (segment (start 218.045 108.571) (end 217.424 107.95) (width 0.25) (layer "F.Cu") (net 8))
 (segment (start 199.22548 78.01978) (end 201.490749 75.754511) (width 0.25) (layer "F.Cu") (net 8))
 (segment (start 225.425 82.612) (end 225.425 87.63) (width 0.25) (layer "F.Cu") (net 9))
 (segment (start 219.71 99.06) (end 219.71 112.508) (width 0.25) (layer "F.Cu") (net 9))
 (segment (start 219.71 99.06) (end 219.71 95.059) (width 0.25) (layer "F.Cu") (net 9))
 (segment (start 219.71 112.508) (end 221.375 114.173) (width 0.25) (layer "F.Cu") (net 9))
 (segment (start 219.646 94.996) (end 220.345 94.996) (width 0.25) (layer "F.Cu") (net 9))
 (segment (start 221.742 91.313) (end 225.425 87.63) (width 0.25) (layer "F.Cu") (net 9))
 (segment (start 220.345 94.996) (end 221.742 93.599) (width 0.25) (layer "F.Cu") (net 9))
 (segment (start 221.742 93.599) (end 221.742 91.313) (width 0.25) (layer "F.Cu") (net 9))
 (segment (start 219.329 78.486) (end 217.17 78.486) (width 0.25) (layer "F.Cu") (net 10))
 (segment (start 202.438 68.58) (end 198.77596 72.24204) (width 0.25) (layer "F.Cu") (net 10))
 (segment (start 236.728 107.1893) (end 236.728 110.25) (width 0.25) (layer "F.Cu") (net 10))
 (segment (start 242.4176 115.7732) (end 242.4176 111.1644) (width 0.25) (layer "F.Cu") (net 10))
 (segment (start 241.6048 110.4392) (end 236.608 110.37) (width 0.25) (layer "F.Cu") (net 10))
 (segment (start 220.092 77.662) (end 219.392 76.962) (width 0.25) (layer "F.Cu") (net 10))
 (segment (start 242.4176 111.1644) (end 241.6048 110.4392) (width 0.25) (layer "F.Cu") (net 10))
 (segment (start 219.392 76.962) (end 219.392 78.423) (width 0.25) (layer "F.Cu") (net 10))
 (segment (start 222.885 77.662) (end 220.092 77.662) (width 0.25) (layer "F.Cu") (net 10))
 (segment (start 217.17 78.486) (end 207.264 68.58) (width 0.25) (layer "F.Cu") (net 10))
 (segment (start 219.392 78.423) (end 219.329 78.486) (width 0.25) (layer "F.Cu") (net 10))
 (segment (start 200.835521 116.394511) (end 240.956111 116.394511) (width 0.25) (layer "F.Cu") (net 10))
 (segment (start 236.728 110.25) (end 236.608 110.37) (width 0.25) (layer "F.Cu") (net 10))
 (segment (start 198.77596 114.33495) (end 200.835521 116.394511) (width 0.25) (layer "F.Cu") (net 10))
 (segment (start 207.264 68.58) (end 202.438 68.58) (width 0.25) (layer "F.Cu") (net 10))
 (segment (start 198.77596 72.24204) (end 198.77596 114.33495) (width 0.25) (layer "F.Cu") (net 10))
 (segment (start 241.796289 116.394511) (end 240.956111 116.394511) (width 0.25) (layer "F.Cu") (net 10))
 (segment (start 236.608 110.37) (end 232.805 114.173) (width 0.25) (layer "F.Cu") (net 10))
 (segment (start 242.4176 115.7732) (end 241.796289 116.394511) (width 0.25) (layer "F.Cu") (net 10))
 (segment (start 224.155 82.612) (end 224.155 82.235928) (width 0.25) (layer "F.Cu") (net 2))
 (segment (start 224.155 82.235928) (end 225.078448 81.31248) (width 0.25) (layer "F.Cu") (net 2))
 (segment (start 212.7237 80.075) (end 212.6687 80.02) (width 0.25) (layer "F.Cu") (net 2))
 (segment (start 227.457 75.819) (end 227.965 76.327) (width 0.25) (layer "F.Cu") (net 2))
 (segment (start 226.06 76.327) (end 226.568 75.819) (width 0.25) (layer "F.Cu") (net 2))
 (segment (start 223.199072 81.28) (end 218.122 81.28) (width 0.25) (layer "F.Cu") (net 2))
 (segment (start 226.568 75.819) (end 227.457 75.819) (width 0.25) (layer "F.Cu") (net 2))
 (segment (start 218.122 81.28) (end 214.312 85.09) (width 0.25) (layer "F.Cu") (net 2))
 (segment (start 212.7237 83.5017) (end 212.7237 80.075) (width 0.25) (layer "F.Cu") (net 2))
 (segment (start 226.06 79.121) (end 226.06 76.327) (width 0.25) (layer "F.Cu") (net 2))
 (segment (start 224.155 82.235928) (end 223.199072 81.28) (width 0.25) (layer "F.Cu") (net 2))
 (segment (start 229.614408 79.68748) (end 232.82398 79.68748) (width 0.25) (layer "F.Cu") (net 2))
 (segment (start 232.82398 79.68748) (end 233.045 79.9085) (width 0.25) (layer "F.Cu") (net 2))
 (segment (start 227.965 78.038072) (end 229.614408 79.68748) (width 0.25) (layer "F.Cu") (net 2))
 (segment (start 227.36248 81.31248) (end 227.965 81.915) (width 0.25) (layer "F.Cu") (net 2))
 (segment (start 209.6108 80.02) (end 209.6008 80.01) (width 0.25) (layer "F.Cu") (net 2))
 (segment (start 227.965 81.026) (end 226.06 79.121) (width 0.25) (layer "F.Cu") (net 2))
 (segment (start 212.6687 80.02) (end 209.6108 80.02) (width 0.25) (layer "F.Cu") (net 2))
 (segment (start 227.965 76.327) (end 227.965 77.662) (width 0.25) (layer "F.Cu") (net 2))
 (segment (start 214.312 85.09) (end 212.7237 83.5017) (width 0.25) (layer "F.Cu") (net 2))
 (segment (start 227.965 82.612) (end 227.965 81.026) (width 0.25) (layer "F.Cu") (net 2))
 (segment (start 227.965 81.915) (end 227.965 82.612) (width 0.25) (layer "F.Cu") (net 2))
 (segment (start 227.965 77.662) (end 227.965 78.038072) (width 0.25) (layer "F.Cu") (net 2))
 (segment (start 225.078448 81.31248) (end 227.36248 81.31248) (width 0.25) (layer "F.Cu") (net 2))
 (segment (start 200.704689 66.135489) (end 206.915489 66.135489) (width 0.25) (layer "F.Cu") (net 14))
 (segment (start 206.915489 66.135489) (end 217.742 76.962) (width 0.25) (layer "F.Cu") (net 14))
 (segment (start 185.035 77.51) (end 189.330178 77.51) (width 0.25) (layer "F.Cu") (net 14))
 (segment (start 183.357 75.832) (end 185.035 77.51) (width 0.25) (layer "F.Cu") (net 14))
 (segment (start 189.330178 77.51) (end 200.704689 66.135489) (width 0.25) (layer "F.Cu") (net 14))
 (segment (start 181.864 75.832) (end 183.357 75.832) (width 0.25) (layer "F.Cu") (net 14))
 (segment (start 215.265 73.025) (end 206.883 64.643) (width 0.25) (layer "F.Cu") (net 15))
 (segment (start 191.135 74.435) (end 190.6 74.97) (width 0.25) (layer "F.Cu") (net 15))
 (segment (start 191.93452 72.11148) (end 199.403 64.643) (width 0.25) (layer "F.Cu") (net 15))
 (segment (start 191.93452 73.63548) (end 191.93452 72.11148) (width 0.25) (layer "F.Cu") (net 15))
 (segment (start 206.883 64.643) (end 199.403 64.643) (width 0.25) (layer "F.Cu") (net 15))
 (segment (start 218.123 73.025) (end 215.265 73.025) (width 0.25) (layer "F.Cu") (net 15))
 (segment (start 190.6 74.97) (end 188.345 74.97) (width 0.25) (layer "F.Cu") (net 15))
 (segment (start 191.135 74.435) (end 191.93452 73.63548) (width 0.25) (layer "F.Cu") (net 15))
 (segment (start 202.815 102.87) (end 205.989022 102.87) (width 0.25) (layer "F.Cu") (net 16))
 (segment (start 213.863022 94.996) (end 217.996 94.996) (width 0.25) (layer "F.Cu") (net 16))
 (segment (start 201.05 101.105) (end 202.815 102.87) (width 0.25) (layer "F.Cu") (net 16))
 (segment (start 205.989022 102.87) (end 213.863022 94.996) (width 0.25) (layer "F.Cu") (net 16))
 (segment (start 200.025 101.105) (end 201.05 101.105) (width 0.25) (layer "F.Cu") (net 16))
 (segment (start 209.042 97.9554) (end 208.4996 97.9554) (width 0.25) (layer "F.Cu") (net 17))
 (segment (start 208.4996 97.9554) (end 206.125 100.33) (width 0.25) (layer "F.Cu") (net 17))
 (segment (start 214.6808 92.71) (end 220.917 92.71) (width 0.25) (layer "F.Cu") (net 17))
 (segment (start 209.4354 97.9554) (end 214.6808 92.71) (width 0.25) (layer "F.Cu") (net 17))
 (segment (start 209.042 97.9554) (end 209.4354 97.9554) (width 0.25) (layer "F.Cu") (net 17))
 (segment (start 209.995489 85.914511) (end 209.995489 87.818211) (width 0.25) (layer "F.Cu") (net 18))
 (segment (start 201.2188 83.357822) (end 201.2188 79.0662) (width 0.25) (layer "F.Cu") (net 18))
 (segment (start 201.2188 79.0662) (end 202.815 77.47) (width 0.25) (layer "F.Cu") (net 18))
 (segment (start 212.662 85.09) (end 211.837489 85.914511) (width 0.25) (layer "F.Cu") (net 18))
 (segment (start 203.775489 85.914511) (end 201.2188 83.357822) (width 0.25) (layer "F.Cu") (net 18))
 (segment (start 209.995489 85.914511) (end 203.775489 85.914511) (width 0.25) (layer "F.Cu") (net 18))
 (segment (start 211.837489 85.914511) (end 209.995489 85.914511) (width 0.25) (layer "F.Cu") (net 18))
 (segment (start 209.995489 87.818211) (end 209.9297 87.884) (width 0.25) (layer "F.Cu") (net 18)))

